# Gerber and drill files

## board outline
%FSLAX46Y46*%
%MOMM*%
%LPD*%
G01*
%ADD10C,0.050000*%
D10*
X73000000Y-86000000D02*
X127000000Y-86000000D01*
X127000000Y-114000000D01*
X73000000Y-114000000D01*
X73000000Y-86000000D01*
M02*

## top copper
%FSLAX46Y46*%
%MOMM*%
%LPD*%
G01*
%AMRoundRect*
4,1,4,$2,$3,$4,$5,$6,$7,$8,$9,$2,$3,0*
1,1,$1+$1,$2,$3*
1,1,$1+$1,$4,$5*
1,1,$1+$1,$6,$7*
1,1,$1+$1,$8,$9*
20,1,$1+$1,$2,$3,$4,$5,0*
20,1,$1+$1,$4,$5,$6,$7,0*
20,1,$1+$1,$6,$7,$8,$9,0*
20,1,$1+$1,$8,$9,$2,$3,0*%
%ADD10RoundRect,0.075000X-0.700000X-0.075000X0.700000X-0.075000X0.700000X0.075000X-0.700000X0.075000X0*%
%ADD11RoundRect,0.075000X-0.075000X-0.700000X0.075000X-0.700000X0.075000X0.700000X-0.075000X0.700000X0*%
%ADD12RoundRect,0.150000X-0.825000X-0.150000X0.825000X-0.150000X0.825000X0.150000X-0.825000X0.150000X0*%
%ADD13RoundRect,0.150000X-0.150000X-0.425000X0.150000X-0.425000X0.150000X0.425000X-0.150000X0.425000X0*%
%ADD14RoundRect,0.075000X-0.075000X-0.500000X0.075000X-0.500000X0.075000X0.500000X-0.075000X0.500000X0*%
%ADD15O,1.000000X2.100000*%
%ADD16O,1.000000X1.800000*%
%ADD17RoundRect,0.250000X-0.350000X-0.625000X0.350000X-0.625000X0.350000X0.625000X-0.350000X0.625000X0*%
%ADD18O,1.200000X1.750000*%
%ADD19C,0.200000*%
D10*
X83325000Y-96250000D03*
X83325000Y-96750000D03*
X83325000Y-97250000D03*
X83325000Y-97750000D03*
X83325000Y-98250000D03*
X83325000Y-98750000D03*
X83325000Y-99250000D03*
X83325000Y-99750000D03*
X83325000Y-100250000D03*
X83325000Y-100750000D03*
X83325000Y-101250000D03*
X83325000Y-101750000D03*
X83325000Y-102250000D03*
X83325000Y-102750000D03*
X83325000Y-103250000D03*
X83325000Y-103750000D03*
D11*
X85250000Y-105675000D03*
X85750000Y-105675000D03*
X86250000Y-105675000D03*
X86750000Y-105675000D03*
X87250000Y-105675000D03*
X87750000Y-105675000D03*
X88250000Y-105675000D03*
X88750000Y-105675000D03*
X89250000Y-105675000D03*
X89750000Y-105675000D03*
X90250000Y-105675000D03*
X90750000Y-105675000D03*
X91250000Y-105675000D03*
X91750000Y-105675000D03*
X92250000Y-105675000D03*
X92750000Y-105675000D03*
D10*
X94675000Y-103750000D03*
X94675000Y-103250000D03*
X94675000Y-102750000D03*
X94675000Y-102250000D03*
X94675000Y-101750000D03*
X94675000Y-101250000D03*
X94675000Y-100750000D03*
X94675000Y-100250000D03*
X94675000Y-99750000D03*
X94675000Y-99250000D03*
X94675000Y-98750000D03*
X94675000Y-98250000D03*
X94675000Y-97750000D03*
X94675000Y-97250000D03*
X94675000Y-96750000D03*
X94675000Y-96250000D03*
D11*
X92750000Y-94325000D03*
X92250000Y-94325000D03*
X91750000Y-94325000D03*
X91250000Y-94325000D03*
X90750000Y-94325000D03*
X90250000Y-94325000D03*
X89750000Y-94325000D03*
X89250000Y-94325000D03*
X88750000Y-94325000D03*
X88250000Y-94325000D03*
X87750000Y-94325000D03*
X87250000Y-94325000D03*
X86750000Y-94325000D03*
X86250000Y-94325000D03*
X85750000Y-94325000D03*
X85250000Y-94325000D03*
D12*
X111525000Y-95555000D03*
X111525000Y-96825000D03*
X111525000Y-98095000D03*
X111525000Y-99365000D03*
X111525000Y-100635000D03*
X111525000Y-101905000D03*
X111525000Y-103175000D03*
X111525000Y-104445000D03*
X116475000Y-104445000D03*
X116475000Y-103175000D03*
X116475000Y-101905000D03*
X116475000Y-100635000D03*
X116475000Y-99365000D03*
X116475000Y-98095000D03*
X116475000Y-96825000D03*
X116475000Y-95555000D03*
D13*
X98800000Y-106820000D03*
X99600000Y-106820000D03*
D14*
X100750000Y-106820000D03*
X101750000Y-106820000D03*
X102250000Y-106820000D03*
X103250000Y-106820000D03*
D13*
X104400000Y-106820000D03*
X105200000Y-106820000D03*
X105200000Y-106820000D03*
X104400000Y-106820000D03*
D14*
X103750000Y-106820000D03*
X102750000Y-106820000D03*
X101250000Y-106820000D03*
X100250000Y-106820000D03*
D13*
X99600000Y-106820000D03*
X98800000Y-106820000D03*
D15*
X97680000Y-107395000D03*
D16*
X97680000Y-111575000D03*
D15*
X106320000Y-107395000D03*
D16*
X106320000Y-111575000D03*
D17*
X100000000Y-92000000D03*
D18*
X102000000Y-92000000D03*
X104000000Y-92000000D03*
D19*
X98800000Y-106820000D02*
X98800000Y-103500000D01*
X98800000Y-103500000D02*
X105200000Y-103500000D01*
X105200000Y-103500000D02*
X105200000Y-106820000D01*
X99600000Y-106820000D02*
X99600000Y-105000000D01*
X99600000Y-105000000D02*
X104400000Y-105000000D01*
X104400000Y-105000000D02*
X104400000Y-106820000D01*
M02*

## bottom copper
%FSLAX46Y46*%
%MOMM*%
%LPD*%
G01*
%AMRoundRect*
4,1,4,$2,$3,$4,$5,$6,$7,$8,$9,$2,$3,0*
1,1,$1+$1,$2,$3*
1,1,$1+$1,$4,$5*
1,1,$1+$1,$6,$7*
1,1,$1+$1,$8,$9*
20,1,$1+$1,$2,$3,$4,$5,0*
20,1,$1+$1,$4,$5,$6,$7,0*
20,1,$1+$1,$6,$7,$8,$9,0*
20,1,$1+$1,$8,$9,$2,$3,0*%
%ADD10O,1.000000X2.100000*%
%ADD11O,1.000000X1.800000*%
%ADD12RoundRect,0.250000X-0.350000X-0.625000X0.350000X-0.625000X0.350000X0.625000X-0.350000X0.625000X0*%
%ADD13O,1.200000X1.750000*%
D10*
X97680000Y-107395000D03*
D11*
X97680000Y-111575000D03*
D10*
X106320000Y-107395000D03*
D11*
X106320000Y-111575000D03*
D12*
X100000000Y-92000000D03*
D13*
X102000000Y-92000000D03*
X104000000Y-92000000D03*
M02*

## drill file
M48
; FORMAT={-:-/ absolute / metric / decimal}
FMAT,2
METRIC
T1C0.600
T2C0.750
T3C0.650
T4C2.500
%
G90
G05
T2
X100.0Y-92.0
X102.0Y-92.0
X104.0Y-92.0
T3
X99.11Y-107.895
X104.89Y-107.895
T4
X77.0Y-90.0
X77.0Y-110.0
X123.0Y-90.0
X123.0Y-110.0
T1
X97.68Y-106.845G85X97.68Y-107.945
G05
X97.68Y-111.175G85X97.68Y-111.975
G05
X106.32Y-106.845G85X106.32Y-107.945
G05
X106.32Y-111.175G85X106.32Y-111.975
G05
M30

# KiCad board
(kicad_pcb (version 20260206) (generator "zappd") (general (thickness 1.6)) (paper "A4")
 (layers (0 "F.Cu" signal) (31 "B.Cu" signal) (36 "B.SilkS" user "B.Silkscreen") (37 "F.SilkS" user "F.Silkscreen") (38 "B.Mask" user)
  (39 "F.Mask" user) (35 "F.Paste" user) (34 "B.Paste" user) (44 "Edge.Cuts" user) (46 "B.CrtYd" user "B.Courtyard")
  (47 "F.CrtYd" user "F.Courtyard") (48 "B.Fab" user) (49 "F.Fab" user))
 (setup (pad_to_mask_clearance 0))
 (gr_rect (start 73.0 86.0) (end 127.0 114.0) (stroke (width 0.05) (type default)) (fill none) (layer "Edge.Cuts"))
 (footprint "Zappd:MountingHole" (layer "F.Cu") (at 77.0 90.0)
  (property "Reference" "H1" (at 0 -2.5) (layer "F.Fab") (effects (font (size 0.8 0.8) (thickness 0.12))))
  (pad "" np_thru_hole circle (at 0 0) (size 2.5 2.5) (drill 2.5) (layers "*.Cu" "*.Mask")))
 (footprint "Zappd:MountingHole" (layer "F.Cu") (at 123.0 90.0)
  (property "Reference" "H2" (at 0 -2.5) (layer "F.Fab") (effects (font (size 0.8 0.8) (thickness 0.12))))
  (pad "" np_thru_hole circle (at 0 0) (size 2.5 2.5) (drill 2.5) (layers "*.Cu" "*.Mask")))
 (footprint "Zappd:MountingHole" (layer "F.Cu") (at 123.0 110.0)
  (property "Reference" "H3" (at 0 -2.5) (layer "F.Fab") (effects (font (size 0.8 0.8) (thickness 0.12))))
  (pad "" np_thru_hole circle (at 0 0) (size 2.5 2.5) (drill 2.5) (layers "*.Cu" "*.Mask")))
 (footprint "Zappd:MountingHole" (layer "F.Cu") (at 77.0 110.0)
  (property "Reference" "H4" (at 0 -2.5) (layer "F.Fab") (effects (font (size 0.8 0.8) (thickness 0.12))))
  (pad "" np_thru_hole circle (at 0 0) (size 2.5 2.5) (drill 2.5) (layers "*.Cu" "*.Mask")))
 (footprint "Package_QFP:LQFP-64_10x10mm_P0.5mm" (layer "F.Cu") (at 89 100)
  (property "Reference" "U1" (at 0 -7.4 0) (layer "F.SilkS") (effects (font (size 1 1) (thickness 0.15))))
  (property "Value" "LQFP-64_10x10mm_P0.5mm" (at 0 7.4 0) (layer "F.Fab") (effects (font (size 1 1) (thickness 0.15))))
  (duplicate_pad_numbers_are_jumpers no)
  (pad "1" smd roundrect (at -5.675 -3.75) (size 1.55 0.3) (layers "F.Cu" "F.Mask" "F.Paste") (roundrect_rratio 0.25))
  (pad "2" smd roundrect (at -5.675 -3.25) (size 1.55 0.3) (layers "F.Cu" "F.Mask" "F.Paste") (roundrect_rratio 0.25))
  (pad "3" smd roundrect (at -5.675 -2.75) (size 1.55 0.3) (layers "F.Cu" "F.Mask" "F.Paste") (roundrect_rratio 0.25))
  (pad "4" smd roundrect (at -5.675 -2.25) (size 1.55 0.3) (layers "F.Cu" "F.Mask" "F.Paste") (roundrect_rratio 0.25))
  (pad "5" smd roundrect (at -5.675 -1.75) (size 1.55 0.3) (layers "F.Cu" "F.Mask" "F.Paste") (roundrect_rratio 0.25))
  (pad "6" smd roundrect (at -5.675 -1.25) (size 1.55 0.3) (layers "F.Cu" "F.Mask" "F.Paste") (roundrect_rratio 0.25))
  (pad "7" smd roundrect (at -5.675 -0.75) (size 1.55 0.3) (layers "F.Cu" "F.Mask" "F.Paste") (roundrect_rratio 0.25))
  (pad "8" smd roundrect (at -5.675 -0.25) (size 1.55 0.3) (layers "F.Cu" "F.Mask" "F.Paste") (roundrect_rratio 0.25))
  (pad "9" smd roundrect (at -5.675 0.25) (size 1.55 0.3) (layers "F.Cu" "F.Mask" "F.Paste") (roundrect_rratio 0.25))
  (pad "10" smd roundrect (at -5.675 0.75) (size 1.55 0.3) (layers "F.Cu" "F.Mask" "F.Paste") (roundrect_rratio 0.25))
  (pad "11" smd roundrect (at -5.675 1.25) (size 1.55 0.3) (layers "F.Cu" "F.Mask" "F.Paste") (roundrect_rratio 0.25))
  (pad "12" smd roundrect (at -5.675 1.75) (size 1.55 0.3) (layers "F.Cu" "F.Mask" "F.Paste") (roundrect_rratio 0.25))
  (pad "13" smd roundrect (at -5.675 2.25) (size 1.55 0.3) (layers "F.Cu" "F.Mask" "F.Paste") (roundrect_rratio 0.25))
  (pad "14" smd roundrect (at -5.675 2.75) (size 1.55 0.3) (layers "F.Cu" "F.Mask" "F.Paste") (roundrect_rratio 0.25))
  (pad "15" smd roundrect (at -5.675 3.25) (size 1.55 0.3) (layers "F.Cu" "F.Mask" "F.Paste") (roundrect_rratio 0.25))
  (pad "16" smd roundrect (at -5.675 3.75) (size 1.55 0.3) (layers "F.Cu" "F.Mask" "F.Paste") (roundrect_rratio 0.25))
  (pad "17" smd roundrect (at -3.75 5.675) (size 0.3 1.55) (layers "F.Cu" "F.Mask" "F.Paste") (roundrect_rratio 0.25))
  (pad "18" smd roundrect (at -3.25 5.675) (size 0.3 1.55) (layers "F.Cu" "F.Mask" "F.Paste") (roundrect_rratio 0.25))
  (pad "19" smd roundrect (at -2.75 5.675) (size 0.3 1.55) (layers "F.Cu" "F.Mask" "F.Paste") (roundrect_rratio 0.25))
  (pad "20" smd roundrect (at -2.25 5.675) (size 0.3 1.55) (layers "F.Cu" "F.Mask" "F.Paste") (roundrect_rratio 0.25))
  (pad "21" smd roundrect (at -1.75 5.675) (size 0.3 1.55) (layers "F.Cu" "F.Mask" "F.Paste") (roundrect_rratio 0.25))
  (pad "22" smd roundrect (at -1.25 5.675) (size 0.3 1.55) (layers "F.Cu" "F.Mask" "F.Paste") (roundrect_rratio 0.25))
  (pad "23" smd roundrect (at -0.75 5.675) (size 0.3 1.55) (layers "F.Cu" "F.Mask" "F.Paste") (roundrect_rratio 0.25))
  (pad "24" smd roundrect (at -0.25 5.675) (size 0.3 1.55) (layers "F.Cu" "F.Mask" "F.Paste") (roundrect_rratio 0.25))
  (pad "25" smd roundrect (at 0.25 5.675) (size 0.3 1.55) (layers "F.Cu" "F.Mask" "F.Paste") (roundrect_rratio 0.25))
  (pad "26" smd roundrect (at 0.75 5.675) (size 0.3 1.55) (layers "F.Cu" "F.Mask" "F.Paste") (roundrect_rratio 0.25))
  (pad "27" smd roundrect (at 1.25 5.675) (size 0.3 1.55) (layers "F.Cu" "F.Mask" "F.Paste") (roundrect_rratio 0.25))
  (pad "28" smd roundrect (at 1.75 5.675) (size 0.3 1.55) (layers "F.Cu" "F.Mask" "F.Paste") (roundrect_rratio 0.25))
  (pad "29" smd roundrect (at 2.25 5.675) (size 0.3 1.55) (layers "F.Cu" "F.Mask" "F.Paste") (roundrect_rratio 0.25))
  (pad "30" smd roundrect (at 2.75 5.675) (size 0.3 1.55) (layers "F.Cu" "F.Mask" "F.Paste") (roundrect_rratio 0.25))
  (pad "31" smd roundrect (at 3.25 5.675) (size 0.3 1.55) (layers "F.Cu" "F.Mask" "F.Paste") (roundrect_rratio 0.25))
  (pad "32" smd roundrect (at 3.75 5.675) (size 0.3 1.55) (layers "F.Cu" "F.Mask" "F.Paste") (roundrect_rratio 0.25))
  (pad "33" smd roundrect (at 5.675 3.75) (size 1.55 0.3) (layers "F.Cu" "F.Mask" "F.Paste") (roundrect_rratio 0.25))
  (pad "34" smd roundrect (at 5.675 3.25) (size 1.55 0.3) (layers "F.Cu" "F.Mask" "F.Paste") (roundrect_rratio 0.25))
  (pad "35" smd roundrect (at 5.675 2.75) (size 1.55 0.3) (layers "F.Cu" "F.Mask" "F.Paste") (roundrect_rratio 0.25))
  (pad "36" smd roundrect (at 5.675 2.25) (size 1.55 0.3) (layers "F.Cu" "F.Mask" "F.Paste") (roundrect_rratio 0.25))
  (pad "37" smd roundrect (at 5.675 1.75) (size 1.55 0.3) (layers "F.Cu" "F.Mask" "F.Paste") (roundrect_rratio 0.25))
  (pad "38" smd roundrect (at 5.675 1.25) (size 1.55 0.3) (layers "F.Cu" "F.Mask" "F.Paste") (roundrect_rratio 0.25))
  (pad "39" smd roundrect (at 5.675 0.75) (size 1.55 0.3) (layers "F.Cu" "F.Mask" "F.Paste") (roundrect_rratio 0.25))
  (pad "40" smd roundrect (at 5.675 0.25) (size 1.55 0.3) (layers "F.Cu" "F.Mask" "F.Paste") (roundrect_rratio 0.25))
  (pad "41" smd roundrect (at 5.675 -0.25) (size 1.55 0.3) (layers "F.Cu" "F.Mask" "F.Paste") (roundrect_rratio 0.25))
  (pad "42" smd roundrect (at 5.675 -0.75) (size 1.55 0.3) (layers "F.Cu" "F.Mask" "F.Paste") (roundrect_rratio 0.25))
  (pad "43" smd roundrect (at 5.675 -1.25) (size 1.55 0.3) (layers "F.Cu" "F.Mask" "F.Paste") (roundrect_rratio 0.25))
  (pad "44" smd roundrect (at 5.675 -1.75) (size 1.55 0.3) (layers "F.Cu" "F.Mask" "F.Paste") (roundrect_rratio 0.25))
  (pad "45" smd roundrect (at 5.675 -2.25) (size 1.55 0.3) (layers "F.Cu" "F.Mask" "F.Paste") (roundrect_rratio 0.25))
  (pad "46" smd roundrect (at 5.675 -2.75) (size 1.55 0.3) (layers "F.Cu" "F.Mask" "F.Paste") (roundrect_rratio 0.25))
  (pad "47" smd roundrect (at 5.675 -3.25) (size 1.55 0.3) (layers "F.Cu" "F.Mask" "F.Paste") (roundrect_rratio 0.25))
  (pad "48" smd roundrect (at 5.675 -3.75) (size 1.55 0.3) (layers "F.Cu" "F.Mask" "F.Paste") (roundrect_rratio 0.25))
  (pad "49" smd roundrect (at 3.75 -5.675) (size 0.3 1.55) (layers "F.Cu" "F.Mask" "F.Paste") (roundrect_rratio 0.25))
  (pad "50" smd roundrect (at 3.25 -5.675) (size 0.3 1.55) (layers "F.Cu" "F.Mask" "F.Paste") (roundrect_rratio 0.25))
  (pad "51" smd roundrect (at 2.75 -5.675) (size 0.3 1.55) (layers "F.Cu" "F.Mask" "F.Paste") (roundrect_rratio 0.25))
  (pad "52" smd roundrect (at 2.25 -5.675) (size 0.3 1.55) (layers "F.Cu" "F.Mask" "F.Paste") (roundrect_rratio 0.25))
  (pad "53" smd roundrect (at 1.75 -5.675) (size 0.3 1.55) (layers "F.Cu" "F.Mask" "F.Paste") (roundrect_rratio 0.25))
  (pad "54" smd roundrect (at 1.25 -5.675) (size 0.3 1.55) (layers "F.Cu" "F.Mask" "F.Paste") (roundrect_rratio 0.25))
  (pad "55" smd roundrect (at 0.75 -5.675) (size 0.3 1.55) (layers "F.Cu" "F.Mask" "F.Paste") (roundrect_rratio 0.25))
  (pad "56" smd roundrect (at 0.25 -5.675) (size 0.3 1.55) (layers "F.Cu" "F.Mask" "F.Paste") (roundrect_rratio 0.25))
  (pad "57" smd roundrect (at -0.25 -5.675) (size 0.3 1.55) (layers "F.Cu" "F.Mask" "F.Paste") (roundrect_rratio 0.25))
  (pad "58" smd roundrect (at -0.75 -5.675) (size 0.3 1.55) (layers "F.Cu" "F.Mask" "F.Paste") (roundrect_rratio 0.25))
  (pad "59" smd roundrect (at -1.25 -5.675) (size 0.3 1.55) (layers "F.Cu" "F.Mask" "F.Paste") (roundrect_rratio 0.25))
  (pad "60" smd roundrect (at -1.75 -5.675) (size 0.3 1.55) (layers "F.Cu" "F.Mask" "F.Paste") (roundrect_rratio 0.25))
  (pad "61" smd roundrect (at -2.25 -5.675) (size 0.3 1.55) (layers "F.Cu" "F.Mask" "F.Paste") (roundrect_rratio 0.25))
  (pad "62" smd roundrect (at -2.75 -5.675) (size 0.3 1.55) (layers "F.Cu" "F.Mask" "F.Paste") (roundrect_rratio 0.25))
  (pad "63" smd roundrect (at -3.25 -5.675) (size 0.3 1.55) (layers "F.Cu" "F.Mask" "F.Paste") (roundrect_rratio 0.25))
  (pad "64" smd roundrect (at -3.75 -5.675) (size 0.3 1.55) (layers "F.Cu" "F.Mask" "F.Paste") (roundrect_rratio 0.25)))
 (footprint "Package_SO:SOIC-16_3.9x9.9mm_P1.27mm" (layer "F.Cu") (at 114 100)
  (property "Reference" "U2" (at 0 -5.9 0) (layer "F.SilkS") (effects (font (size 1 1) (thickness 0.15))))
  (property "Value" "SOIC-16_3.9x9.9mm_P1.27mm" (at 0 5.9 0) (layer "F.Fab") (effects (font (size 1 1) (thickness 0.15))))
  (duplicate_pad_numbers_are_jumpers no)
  (pad "1" smd roundrect (at -2.475 -4.445) (size 1.95 0.6) (layers "F.Cu" "F.Mask" "F.Paste") (roundrect_rratio 0.25))
  (pad "2" smd roundrect (at -2.475 -3.175) (size 1.95 0.6) (layers "F.Cu" "F.Mask" "F.Paste") (roundrect_rratio 0.25))
  (pad "3" smd roundrect (at -2.475 -1.905) (size 1.95 0.6) (layers "F.Cu" "F.Mask" "F.Paste") (roundrect_rratio 0.25))
  (pad "4" smd roundrect (at -2.475 -0.635) (size 1.95 0.6) (layers "F.Cu" "F.Mask" "F.Paste") (roundrect_rratio 0.25))
  (pad "5" smd roundrect (at -2.475 0.635) (size 1.95 0.6) (layers "F.Cu" "F.Mask" "F.Paste") (roundrect_rratio 0.25))
  (pad "6" smd roundrect (at -2.475 1.905) (size 1.95 0.6) (layers "F.Cu" "F.Mask" "F.Paste") (roundrect_rratio 0.25))
  (pad "7" smd roundrect (at -2.475 3.175) (size 1.95 0.6) (layers "F.Cu" "F.Mask" "F.Paste") (roundrect_rratio 0.25))
  (pad "8" smd roundrect (at -2.475 4.445) (size 1.95 0.6) (layers "F.Cu" "F.Mask" "F.Paste") (roundrect_rratio 0.25))
  (pad "9" smd roundrect (at 2.475 4.445) (size 1.95 0.6) (layers "F.Cu" "F.Mask" "F.Paste") (roundrect_rratio 0.25))
  (pad "10" smd roundrect (at 2.475 3.175) (size 1.95 0.6) (layers "F.Cu" "F.Mask" "F.Paste") (roundrect_rratio 0.25))
  (pad "11" smd roundrect (at 2.475 1.905) (size 1.95 0.6) (layers "F.Cu" "F.Mask" "F.Paste") (roundrect_rratio 0.25))
  (pad "12" smd roundrect (at 2.475 0.635) (size 1.95 0.6) (layers "F.Cu" "F.Mask" "F.Paste") (roundrect_rratio 0.25))
  (pad "13" smd roundrect (at 2.475 -0.635) (size 1.95 0.6) (layers "F.Cu" "F.Mask" "F.Paste") (roundrect_rratio 0.25))
  (pad "14" smd roundrect (at 2.475 -1.905) (size 1.95 0.6) (layers "F.Cu" "F.Mask" "F.Paste") (roundrect_rratio 0.25))
  (pad "15" smd roundrect (at 2.475 -3.175) (size 1.95 0.6) (layers "F.Cu" "F.Mask" "F.Paste") (roundrect_rratio 0.25))
  (pad "16" smd roundrect (at 2.475 -4.445) (size 1.95 0.6) (layers "F.Cu" "F.Mask" "F.Paste") (roundrect_rratio 0.25)))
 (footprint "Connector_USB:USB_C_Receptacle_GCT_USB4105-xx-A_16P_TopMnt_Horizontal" (layer "F.Cu") (at 102 110.5)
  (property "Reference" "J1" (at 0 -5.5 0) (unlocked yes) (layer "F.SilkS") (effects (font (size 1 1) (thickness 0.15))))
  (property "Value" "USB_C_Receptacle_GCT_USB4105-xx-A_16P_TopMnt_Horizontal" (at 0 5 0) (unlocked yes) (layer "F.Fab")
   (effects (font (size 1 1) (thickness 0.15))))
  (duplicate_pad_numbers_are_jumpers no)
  (pad "" np_thru_hole circle (at -2.89 -2.605) (size 0.65 0.65) (drill 0.65) (layers "*.Cu" "*.Mask"))
  (pad "" np_thru_hole circle (at 2.89 -2.605) (size 0.65 0.65) (drill 0.65) (layers "*.Cu" "*.Mask"))
  (pad "A1" smd roundrect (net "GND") (at -3.2 -3.68) (size 0.6 1.15) (layers "F.Cu" "F.Mask" "F.Paste") (roundrect_rratio 0.25))
  (pad "A4" smd roundrect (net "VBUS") (at -2.4 -3.68) (size 0.6 1.15) (layers "F.Cu" "F.Mask" "F.Paste") (roundrect_rratio 0.25))
  (pad "A5" smd roundrect (at -1.25 -3.68) (size 0.3 1.15) (layers "F.Cu" "F.Mask" "F.Paste") (roundrect_rratio 0.25))
  (pad "A6" smd roundrect (at -0.25 -3.68) (size 0.3 1.15) (layers "F.Cu" "F.Mask" "F.Paste") (roundrect_rratio 0.25))
  (pad "A7" smd roundrect (at 0.25 -3.68) (size 0.3 1.15) (layers "F.Cu" "F.Mask" "F.Paste") (roundrect_rratio 0.25))
  (pad "A8" smd roundrect (at 1.25 -3.68) (size 0.3 1.15) (layers "F.Cu" "F.Mask" "F.Paste") (roundrect_rratio 0.25))
  (pad "A9" smd roundrect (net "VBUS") (at 2.4 -3.68) (size 0.6 1.15) (layers "F.Cu" "F.Mask" "F.Paste") (roundrect_rratio 0.25))
  (pad "A12" smd roundrect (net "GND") (at 3.2 -3.68) (size 0.6 1.15) (layers "F.Cu" "F.Mask" "F.Paste") (roundrect_rratio 0.25))
  (pad "B1" smd roundrect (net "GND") (at 3.2 -3.68) (size 0.6 1.15) (layers "F.Cu" "F.Mask" "F.Paste") (roundrect_rratio 0.25))
  (pad "B4" smd roundrect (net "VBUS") (at 2.4 -3.68) (size 0.6 1.15) (layers "F.Cu" "F.Mask" "F.Paste") (roundrect_rratio 0.25))
  (pad "B5" smd roundrect (at 1.75 -3.68) (size 0.3 1.15) (layers "F.Cu" "F.Mask" "F.Paste") (roundrect_rratio 0.25))
  (pad "B6" smd roundrect (at 0.75 -3.68) (size 0.3 1.15) (layers "F.Cu" "F.Mask" "F.Paste") (roundrect_rratio 0.25))
  (pad "B7" smd roundrect (at -0.75 -3.68) (size 0.3 1.15) (layers "F.Cu" "F.Mask" "F.Paste") (roundrect_rratio 0.25))
  (pad "B8" smd roundrect (at -1.75 -3.68) (size 0.3 1.15) (layers "F.Cu" "F.Mask" "F.Paste") (roundrect_rratio 0.25))
  (pad "B9" smd roundrect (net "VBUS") (at -2.4 -3.68) (size 0.6 1.15) (layers "F.Cu" "F.Mask" "F.Paste") (roundrect_rratio 0.25))
  (pad "B12" smd roundrect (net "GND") (at -3.2 -3.68) (size 0.6 1.15) (layers "F.Cu" "F.Mask" "F.Paste") (roundrect_rratio 0.25))
  (pad "SH" thru_hole oval (at -4.32 -3.105) (size 1 2.1) (drill oval 0.6 1.7) (layers "*.Cu" "*.Mask" "F.Paste") (remove_unused_layers no))
  (pad "SH" thru_hole oval (at -4.32 1.075) (size 1 1.8) (drill oval 0.6 1.4) (layers "*.Cu" "*.Mask" "F.Paste") (remove_unused_layers no))
  (pad "SH" thru_hole oval (at 4.32 -3.105) (size 1 2.1) (drill oval 0.6 1.7) (layers "*.Cu" "*.Mask" "F.Paste") (remove_unused_layers no))
  (pad "SH" thru_hole oval (at 4.32 1.075) (size 1 1.8) (drill oval 0.6 1.4) (layers "*.Cu" "*.Mask" "F.Paste") (remove_unused_layers no)))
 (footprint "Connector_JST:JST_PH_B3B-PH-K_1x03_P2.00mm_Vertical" (layer "F.Cu") (at 100 92)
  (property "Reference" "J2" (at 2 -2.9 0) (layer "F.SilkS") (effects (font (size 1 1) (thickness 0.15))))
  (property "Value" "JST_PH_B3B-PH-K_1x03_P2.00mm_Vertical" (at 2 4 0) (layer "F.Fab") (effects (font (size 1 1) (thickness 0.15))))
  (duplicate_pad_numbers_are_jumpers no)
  (pad "1" thru_hole roundrect (at 0 0) (size 1.2 1.75) (drill 0.75) (layers "*.Cu" "*.Mask") (remove_unused_layers no)
   (roundrect_rratio 0.208333))
  (pad "2" thru_hole oval (at 2 0) (size 1.2 1.75) (drill 0.75) (layers "*.Cu" "*.Mask") (remove_unused_layers no))
  (pad "3" thru_hole oval (at 4 0) (size 1.2 1.75) (drill 0.75) (layers "*.Cu" "*.Mask") (remove_unused_layers no)))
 (segment (start 98.8000 106.8200) (end 98.8000 103.5000) (width 0.2) (layer "F.Cu") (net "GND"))
 (segment (start 98.8000 103.5000) (end 105.2000 103.5000) (width 0.2) (layer "F.Cu") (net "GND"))
 (segment (start 105.2000 103.5000) (end 105.2000 106.8200) (width 0.2) (layer "F.Cu") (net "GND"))
 (segment (start 99.6000 106.8200) (end 99.6000 105.0000) (width 0.2) (layer "F.Cu") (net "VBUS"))
 (segment (start 99.6000 105.0000) (end 104.4000 105.0000) (width 0.2) (layer "F.Cu") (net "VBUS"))
 (segment (start 104.4000 105.0000) (end 104.4000 106.8200) (width 0.2) (layer "F.Cu") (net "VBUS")))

